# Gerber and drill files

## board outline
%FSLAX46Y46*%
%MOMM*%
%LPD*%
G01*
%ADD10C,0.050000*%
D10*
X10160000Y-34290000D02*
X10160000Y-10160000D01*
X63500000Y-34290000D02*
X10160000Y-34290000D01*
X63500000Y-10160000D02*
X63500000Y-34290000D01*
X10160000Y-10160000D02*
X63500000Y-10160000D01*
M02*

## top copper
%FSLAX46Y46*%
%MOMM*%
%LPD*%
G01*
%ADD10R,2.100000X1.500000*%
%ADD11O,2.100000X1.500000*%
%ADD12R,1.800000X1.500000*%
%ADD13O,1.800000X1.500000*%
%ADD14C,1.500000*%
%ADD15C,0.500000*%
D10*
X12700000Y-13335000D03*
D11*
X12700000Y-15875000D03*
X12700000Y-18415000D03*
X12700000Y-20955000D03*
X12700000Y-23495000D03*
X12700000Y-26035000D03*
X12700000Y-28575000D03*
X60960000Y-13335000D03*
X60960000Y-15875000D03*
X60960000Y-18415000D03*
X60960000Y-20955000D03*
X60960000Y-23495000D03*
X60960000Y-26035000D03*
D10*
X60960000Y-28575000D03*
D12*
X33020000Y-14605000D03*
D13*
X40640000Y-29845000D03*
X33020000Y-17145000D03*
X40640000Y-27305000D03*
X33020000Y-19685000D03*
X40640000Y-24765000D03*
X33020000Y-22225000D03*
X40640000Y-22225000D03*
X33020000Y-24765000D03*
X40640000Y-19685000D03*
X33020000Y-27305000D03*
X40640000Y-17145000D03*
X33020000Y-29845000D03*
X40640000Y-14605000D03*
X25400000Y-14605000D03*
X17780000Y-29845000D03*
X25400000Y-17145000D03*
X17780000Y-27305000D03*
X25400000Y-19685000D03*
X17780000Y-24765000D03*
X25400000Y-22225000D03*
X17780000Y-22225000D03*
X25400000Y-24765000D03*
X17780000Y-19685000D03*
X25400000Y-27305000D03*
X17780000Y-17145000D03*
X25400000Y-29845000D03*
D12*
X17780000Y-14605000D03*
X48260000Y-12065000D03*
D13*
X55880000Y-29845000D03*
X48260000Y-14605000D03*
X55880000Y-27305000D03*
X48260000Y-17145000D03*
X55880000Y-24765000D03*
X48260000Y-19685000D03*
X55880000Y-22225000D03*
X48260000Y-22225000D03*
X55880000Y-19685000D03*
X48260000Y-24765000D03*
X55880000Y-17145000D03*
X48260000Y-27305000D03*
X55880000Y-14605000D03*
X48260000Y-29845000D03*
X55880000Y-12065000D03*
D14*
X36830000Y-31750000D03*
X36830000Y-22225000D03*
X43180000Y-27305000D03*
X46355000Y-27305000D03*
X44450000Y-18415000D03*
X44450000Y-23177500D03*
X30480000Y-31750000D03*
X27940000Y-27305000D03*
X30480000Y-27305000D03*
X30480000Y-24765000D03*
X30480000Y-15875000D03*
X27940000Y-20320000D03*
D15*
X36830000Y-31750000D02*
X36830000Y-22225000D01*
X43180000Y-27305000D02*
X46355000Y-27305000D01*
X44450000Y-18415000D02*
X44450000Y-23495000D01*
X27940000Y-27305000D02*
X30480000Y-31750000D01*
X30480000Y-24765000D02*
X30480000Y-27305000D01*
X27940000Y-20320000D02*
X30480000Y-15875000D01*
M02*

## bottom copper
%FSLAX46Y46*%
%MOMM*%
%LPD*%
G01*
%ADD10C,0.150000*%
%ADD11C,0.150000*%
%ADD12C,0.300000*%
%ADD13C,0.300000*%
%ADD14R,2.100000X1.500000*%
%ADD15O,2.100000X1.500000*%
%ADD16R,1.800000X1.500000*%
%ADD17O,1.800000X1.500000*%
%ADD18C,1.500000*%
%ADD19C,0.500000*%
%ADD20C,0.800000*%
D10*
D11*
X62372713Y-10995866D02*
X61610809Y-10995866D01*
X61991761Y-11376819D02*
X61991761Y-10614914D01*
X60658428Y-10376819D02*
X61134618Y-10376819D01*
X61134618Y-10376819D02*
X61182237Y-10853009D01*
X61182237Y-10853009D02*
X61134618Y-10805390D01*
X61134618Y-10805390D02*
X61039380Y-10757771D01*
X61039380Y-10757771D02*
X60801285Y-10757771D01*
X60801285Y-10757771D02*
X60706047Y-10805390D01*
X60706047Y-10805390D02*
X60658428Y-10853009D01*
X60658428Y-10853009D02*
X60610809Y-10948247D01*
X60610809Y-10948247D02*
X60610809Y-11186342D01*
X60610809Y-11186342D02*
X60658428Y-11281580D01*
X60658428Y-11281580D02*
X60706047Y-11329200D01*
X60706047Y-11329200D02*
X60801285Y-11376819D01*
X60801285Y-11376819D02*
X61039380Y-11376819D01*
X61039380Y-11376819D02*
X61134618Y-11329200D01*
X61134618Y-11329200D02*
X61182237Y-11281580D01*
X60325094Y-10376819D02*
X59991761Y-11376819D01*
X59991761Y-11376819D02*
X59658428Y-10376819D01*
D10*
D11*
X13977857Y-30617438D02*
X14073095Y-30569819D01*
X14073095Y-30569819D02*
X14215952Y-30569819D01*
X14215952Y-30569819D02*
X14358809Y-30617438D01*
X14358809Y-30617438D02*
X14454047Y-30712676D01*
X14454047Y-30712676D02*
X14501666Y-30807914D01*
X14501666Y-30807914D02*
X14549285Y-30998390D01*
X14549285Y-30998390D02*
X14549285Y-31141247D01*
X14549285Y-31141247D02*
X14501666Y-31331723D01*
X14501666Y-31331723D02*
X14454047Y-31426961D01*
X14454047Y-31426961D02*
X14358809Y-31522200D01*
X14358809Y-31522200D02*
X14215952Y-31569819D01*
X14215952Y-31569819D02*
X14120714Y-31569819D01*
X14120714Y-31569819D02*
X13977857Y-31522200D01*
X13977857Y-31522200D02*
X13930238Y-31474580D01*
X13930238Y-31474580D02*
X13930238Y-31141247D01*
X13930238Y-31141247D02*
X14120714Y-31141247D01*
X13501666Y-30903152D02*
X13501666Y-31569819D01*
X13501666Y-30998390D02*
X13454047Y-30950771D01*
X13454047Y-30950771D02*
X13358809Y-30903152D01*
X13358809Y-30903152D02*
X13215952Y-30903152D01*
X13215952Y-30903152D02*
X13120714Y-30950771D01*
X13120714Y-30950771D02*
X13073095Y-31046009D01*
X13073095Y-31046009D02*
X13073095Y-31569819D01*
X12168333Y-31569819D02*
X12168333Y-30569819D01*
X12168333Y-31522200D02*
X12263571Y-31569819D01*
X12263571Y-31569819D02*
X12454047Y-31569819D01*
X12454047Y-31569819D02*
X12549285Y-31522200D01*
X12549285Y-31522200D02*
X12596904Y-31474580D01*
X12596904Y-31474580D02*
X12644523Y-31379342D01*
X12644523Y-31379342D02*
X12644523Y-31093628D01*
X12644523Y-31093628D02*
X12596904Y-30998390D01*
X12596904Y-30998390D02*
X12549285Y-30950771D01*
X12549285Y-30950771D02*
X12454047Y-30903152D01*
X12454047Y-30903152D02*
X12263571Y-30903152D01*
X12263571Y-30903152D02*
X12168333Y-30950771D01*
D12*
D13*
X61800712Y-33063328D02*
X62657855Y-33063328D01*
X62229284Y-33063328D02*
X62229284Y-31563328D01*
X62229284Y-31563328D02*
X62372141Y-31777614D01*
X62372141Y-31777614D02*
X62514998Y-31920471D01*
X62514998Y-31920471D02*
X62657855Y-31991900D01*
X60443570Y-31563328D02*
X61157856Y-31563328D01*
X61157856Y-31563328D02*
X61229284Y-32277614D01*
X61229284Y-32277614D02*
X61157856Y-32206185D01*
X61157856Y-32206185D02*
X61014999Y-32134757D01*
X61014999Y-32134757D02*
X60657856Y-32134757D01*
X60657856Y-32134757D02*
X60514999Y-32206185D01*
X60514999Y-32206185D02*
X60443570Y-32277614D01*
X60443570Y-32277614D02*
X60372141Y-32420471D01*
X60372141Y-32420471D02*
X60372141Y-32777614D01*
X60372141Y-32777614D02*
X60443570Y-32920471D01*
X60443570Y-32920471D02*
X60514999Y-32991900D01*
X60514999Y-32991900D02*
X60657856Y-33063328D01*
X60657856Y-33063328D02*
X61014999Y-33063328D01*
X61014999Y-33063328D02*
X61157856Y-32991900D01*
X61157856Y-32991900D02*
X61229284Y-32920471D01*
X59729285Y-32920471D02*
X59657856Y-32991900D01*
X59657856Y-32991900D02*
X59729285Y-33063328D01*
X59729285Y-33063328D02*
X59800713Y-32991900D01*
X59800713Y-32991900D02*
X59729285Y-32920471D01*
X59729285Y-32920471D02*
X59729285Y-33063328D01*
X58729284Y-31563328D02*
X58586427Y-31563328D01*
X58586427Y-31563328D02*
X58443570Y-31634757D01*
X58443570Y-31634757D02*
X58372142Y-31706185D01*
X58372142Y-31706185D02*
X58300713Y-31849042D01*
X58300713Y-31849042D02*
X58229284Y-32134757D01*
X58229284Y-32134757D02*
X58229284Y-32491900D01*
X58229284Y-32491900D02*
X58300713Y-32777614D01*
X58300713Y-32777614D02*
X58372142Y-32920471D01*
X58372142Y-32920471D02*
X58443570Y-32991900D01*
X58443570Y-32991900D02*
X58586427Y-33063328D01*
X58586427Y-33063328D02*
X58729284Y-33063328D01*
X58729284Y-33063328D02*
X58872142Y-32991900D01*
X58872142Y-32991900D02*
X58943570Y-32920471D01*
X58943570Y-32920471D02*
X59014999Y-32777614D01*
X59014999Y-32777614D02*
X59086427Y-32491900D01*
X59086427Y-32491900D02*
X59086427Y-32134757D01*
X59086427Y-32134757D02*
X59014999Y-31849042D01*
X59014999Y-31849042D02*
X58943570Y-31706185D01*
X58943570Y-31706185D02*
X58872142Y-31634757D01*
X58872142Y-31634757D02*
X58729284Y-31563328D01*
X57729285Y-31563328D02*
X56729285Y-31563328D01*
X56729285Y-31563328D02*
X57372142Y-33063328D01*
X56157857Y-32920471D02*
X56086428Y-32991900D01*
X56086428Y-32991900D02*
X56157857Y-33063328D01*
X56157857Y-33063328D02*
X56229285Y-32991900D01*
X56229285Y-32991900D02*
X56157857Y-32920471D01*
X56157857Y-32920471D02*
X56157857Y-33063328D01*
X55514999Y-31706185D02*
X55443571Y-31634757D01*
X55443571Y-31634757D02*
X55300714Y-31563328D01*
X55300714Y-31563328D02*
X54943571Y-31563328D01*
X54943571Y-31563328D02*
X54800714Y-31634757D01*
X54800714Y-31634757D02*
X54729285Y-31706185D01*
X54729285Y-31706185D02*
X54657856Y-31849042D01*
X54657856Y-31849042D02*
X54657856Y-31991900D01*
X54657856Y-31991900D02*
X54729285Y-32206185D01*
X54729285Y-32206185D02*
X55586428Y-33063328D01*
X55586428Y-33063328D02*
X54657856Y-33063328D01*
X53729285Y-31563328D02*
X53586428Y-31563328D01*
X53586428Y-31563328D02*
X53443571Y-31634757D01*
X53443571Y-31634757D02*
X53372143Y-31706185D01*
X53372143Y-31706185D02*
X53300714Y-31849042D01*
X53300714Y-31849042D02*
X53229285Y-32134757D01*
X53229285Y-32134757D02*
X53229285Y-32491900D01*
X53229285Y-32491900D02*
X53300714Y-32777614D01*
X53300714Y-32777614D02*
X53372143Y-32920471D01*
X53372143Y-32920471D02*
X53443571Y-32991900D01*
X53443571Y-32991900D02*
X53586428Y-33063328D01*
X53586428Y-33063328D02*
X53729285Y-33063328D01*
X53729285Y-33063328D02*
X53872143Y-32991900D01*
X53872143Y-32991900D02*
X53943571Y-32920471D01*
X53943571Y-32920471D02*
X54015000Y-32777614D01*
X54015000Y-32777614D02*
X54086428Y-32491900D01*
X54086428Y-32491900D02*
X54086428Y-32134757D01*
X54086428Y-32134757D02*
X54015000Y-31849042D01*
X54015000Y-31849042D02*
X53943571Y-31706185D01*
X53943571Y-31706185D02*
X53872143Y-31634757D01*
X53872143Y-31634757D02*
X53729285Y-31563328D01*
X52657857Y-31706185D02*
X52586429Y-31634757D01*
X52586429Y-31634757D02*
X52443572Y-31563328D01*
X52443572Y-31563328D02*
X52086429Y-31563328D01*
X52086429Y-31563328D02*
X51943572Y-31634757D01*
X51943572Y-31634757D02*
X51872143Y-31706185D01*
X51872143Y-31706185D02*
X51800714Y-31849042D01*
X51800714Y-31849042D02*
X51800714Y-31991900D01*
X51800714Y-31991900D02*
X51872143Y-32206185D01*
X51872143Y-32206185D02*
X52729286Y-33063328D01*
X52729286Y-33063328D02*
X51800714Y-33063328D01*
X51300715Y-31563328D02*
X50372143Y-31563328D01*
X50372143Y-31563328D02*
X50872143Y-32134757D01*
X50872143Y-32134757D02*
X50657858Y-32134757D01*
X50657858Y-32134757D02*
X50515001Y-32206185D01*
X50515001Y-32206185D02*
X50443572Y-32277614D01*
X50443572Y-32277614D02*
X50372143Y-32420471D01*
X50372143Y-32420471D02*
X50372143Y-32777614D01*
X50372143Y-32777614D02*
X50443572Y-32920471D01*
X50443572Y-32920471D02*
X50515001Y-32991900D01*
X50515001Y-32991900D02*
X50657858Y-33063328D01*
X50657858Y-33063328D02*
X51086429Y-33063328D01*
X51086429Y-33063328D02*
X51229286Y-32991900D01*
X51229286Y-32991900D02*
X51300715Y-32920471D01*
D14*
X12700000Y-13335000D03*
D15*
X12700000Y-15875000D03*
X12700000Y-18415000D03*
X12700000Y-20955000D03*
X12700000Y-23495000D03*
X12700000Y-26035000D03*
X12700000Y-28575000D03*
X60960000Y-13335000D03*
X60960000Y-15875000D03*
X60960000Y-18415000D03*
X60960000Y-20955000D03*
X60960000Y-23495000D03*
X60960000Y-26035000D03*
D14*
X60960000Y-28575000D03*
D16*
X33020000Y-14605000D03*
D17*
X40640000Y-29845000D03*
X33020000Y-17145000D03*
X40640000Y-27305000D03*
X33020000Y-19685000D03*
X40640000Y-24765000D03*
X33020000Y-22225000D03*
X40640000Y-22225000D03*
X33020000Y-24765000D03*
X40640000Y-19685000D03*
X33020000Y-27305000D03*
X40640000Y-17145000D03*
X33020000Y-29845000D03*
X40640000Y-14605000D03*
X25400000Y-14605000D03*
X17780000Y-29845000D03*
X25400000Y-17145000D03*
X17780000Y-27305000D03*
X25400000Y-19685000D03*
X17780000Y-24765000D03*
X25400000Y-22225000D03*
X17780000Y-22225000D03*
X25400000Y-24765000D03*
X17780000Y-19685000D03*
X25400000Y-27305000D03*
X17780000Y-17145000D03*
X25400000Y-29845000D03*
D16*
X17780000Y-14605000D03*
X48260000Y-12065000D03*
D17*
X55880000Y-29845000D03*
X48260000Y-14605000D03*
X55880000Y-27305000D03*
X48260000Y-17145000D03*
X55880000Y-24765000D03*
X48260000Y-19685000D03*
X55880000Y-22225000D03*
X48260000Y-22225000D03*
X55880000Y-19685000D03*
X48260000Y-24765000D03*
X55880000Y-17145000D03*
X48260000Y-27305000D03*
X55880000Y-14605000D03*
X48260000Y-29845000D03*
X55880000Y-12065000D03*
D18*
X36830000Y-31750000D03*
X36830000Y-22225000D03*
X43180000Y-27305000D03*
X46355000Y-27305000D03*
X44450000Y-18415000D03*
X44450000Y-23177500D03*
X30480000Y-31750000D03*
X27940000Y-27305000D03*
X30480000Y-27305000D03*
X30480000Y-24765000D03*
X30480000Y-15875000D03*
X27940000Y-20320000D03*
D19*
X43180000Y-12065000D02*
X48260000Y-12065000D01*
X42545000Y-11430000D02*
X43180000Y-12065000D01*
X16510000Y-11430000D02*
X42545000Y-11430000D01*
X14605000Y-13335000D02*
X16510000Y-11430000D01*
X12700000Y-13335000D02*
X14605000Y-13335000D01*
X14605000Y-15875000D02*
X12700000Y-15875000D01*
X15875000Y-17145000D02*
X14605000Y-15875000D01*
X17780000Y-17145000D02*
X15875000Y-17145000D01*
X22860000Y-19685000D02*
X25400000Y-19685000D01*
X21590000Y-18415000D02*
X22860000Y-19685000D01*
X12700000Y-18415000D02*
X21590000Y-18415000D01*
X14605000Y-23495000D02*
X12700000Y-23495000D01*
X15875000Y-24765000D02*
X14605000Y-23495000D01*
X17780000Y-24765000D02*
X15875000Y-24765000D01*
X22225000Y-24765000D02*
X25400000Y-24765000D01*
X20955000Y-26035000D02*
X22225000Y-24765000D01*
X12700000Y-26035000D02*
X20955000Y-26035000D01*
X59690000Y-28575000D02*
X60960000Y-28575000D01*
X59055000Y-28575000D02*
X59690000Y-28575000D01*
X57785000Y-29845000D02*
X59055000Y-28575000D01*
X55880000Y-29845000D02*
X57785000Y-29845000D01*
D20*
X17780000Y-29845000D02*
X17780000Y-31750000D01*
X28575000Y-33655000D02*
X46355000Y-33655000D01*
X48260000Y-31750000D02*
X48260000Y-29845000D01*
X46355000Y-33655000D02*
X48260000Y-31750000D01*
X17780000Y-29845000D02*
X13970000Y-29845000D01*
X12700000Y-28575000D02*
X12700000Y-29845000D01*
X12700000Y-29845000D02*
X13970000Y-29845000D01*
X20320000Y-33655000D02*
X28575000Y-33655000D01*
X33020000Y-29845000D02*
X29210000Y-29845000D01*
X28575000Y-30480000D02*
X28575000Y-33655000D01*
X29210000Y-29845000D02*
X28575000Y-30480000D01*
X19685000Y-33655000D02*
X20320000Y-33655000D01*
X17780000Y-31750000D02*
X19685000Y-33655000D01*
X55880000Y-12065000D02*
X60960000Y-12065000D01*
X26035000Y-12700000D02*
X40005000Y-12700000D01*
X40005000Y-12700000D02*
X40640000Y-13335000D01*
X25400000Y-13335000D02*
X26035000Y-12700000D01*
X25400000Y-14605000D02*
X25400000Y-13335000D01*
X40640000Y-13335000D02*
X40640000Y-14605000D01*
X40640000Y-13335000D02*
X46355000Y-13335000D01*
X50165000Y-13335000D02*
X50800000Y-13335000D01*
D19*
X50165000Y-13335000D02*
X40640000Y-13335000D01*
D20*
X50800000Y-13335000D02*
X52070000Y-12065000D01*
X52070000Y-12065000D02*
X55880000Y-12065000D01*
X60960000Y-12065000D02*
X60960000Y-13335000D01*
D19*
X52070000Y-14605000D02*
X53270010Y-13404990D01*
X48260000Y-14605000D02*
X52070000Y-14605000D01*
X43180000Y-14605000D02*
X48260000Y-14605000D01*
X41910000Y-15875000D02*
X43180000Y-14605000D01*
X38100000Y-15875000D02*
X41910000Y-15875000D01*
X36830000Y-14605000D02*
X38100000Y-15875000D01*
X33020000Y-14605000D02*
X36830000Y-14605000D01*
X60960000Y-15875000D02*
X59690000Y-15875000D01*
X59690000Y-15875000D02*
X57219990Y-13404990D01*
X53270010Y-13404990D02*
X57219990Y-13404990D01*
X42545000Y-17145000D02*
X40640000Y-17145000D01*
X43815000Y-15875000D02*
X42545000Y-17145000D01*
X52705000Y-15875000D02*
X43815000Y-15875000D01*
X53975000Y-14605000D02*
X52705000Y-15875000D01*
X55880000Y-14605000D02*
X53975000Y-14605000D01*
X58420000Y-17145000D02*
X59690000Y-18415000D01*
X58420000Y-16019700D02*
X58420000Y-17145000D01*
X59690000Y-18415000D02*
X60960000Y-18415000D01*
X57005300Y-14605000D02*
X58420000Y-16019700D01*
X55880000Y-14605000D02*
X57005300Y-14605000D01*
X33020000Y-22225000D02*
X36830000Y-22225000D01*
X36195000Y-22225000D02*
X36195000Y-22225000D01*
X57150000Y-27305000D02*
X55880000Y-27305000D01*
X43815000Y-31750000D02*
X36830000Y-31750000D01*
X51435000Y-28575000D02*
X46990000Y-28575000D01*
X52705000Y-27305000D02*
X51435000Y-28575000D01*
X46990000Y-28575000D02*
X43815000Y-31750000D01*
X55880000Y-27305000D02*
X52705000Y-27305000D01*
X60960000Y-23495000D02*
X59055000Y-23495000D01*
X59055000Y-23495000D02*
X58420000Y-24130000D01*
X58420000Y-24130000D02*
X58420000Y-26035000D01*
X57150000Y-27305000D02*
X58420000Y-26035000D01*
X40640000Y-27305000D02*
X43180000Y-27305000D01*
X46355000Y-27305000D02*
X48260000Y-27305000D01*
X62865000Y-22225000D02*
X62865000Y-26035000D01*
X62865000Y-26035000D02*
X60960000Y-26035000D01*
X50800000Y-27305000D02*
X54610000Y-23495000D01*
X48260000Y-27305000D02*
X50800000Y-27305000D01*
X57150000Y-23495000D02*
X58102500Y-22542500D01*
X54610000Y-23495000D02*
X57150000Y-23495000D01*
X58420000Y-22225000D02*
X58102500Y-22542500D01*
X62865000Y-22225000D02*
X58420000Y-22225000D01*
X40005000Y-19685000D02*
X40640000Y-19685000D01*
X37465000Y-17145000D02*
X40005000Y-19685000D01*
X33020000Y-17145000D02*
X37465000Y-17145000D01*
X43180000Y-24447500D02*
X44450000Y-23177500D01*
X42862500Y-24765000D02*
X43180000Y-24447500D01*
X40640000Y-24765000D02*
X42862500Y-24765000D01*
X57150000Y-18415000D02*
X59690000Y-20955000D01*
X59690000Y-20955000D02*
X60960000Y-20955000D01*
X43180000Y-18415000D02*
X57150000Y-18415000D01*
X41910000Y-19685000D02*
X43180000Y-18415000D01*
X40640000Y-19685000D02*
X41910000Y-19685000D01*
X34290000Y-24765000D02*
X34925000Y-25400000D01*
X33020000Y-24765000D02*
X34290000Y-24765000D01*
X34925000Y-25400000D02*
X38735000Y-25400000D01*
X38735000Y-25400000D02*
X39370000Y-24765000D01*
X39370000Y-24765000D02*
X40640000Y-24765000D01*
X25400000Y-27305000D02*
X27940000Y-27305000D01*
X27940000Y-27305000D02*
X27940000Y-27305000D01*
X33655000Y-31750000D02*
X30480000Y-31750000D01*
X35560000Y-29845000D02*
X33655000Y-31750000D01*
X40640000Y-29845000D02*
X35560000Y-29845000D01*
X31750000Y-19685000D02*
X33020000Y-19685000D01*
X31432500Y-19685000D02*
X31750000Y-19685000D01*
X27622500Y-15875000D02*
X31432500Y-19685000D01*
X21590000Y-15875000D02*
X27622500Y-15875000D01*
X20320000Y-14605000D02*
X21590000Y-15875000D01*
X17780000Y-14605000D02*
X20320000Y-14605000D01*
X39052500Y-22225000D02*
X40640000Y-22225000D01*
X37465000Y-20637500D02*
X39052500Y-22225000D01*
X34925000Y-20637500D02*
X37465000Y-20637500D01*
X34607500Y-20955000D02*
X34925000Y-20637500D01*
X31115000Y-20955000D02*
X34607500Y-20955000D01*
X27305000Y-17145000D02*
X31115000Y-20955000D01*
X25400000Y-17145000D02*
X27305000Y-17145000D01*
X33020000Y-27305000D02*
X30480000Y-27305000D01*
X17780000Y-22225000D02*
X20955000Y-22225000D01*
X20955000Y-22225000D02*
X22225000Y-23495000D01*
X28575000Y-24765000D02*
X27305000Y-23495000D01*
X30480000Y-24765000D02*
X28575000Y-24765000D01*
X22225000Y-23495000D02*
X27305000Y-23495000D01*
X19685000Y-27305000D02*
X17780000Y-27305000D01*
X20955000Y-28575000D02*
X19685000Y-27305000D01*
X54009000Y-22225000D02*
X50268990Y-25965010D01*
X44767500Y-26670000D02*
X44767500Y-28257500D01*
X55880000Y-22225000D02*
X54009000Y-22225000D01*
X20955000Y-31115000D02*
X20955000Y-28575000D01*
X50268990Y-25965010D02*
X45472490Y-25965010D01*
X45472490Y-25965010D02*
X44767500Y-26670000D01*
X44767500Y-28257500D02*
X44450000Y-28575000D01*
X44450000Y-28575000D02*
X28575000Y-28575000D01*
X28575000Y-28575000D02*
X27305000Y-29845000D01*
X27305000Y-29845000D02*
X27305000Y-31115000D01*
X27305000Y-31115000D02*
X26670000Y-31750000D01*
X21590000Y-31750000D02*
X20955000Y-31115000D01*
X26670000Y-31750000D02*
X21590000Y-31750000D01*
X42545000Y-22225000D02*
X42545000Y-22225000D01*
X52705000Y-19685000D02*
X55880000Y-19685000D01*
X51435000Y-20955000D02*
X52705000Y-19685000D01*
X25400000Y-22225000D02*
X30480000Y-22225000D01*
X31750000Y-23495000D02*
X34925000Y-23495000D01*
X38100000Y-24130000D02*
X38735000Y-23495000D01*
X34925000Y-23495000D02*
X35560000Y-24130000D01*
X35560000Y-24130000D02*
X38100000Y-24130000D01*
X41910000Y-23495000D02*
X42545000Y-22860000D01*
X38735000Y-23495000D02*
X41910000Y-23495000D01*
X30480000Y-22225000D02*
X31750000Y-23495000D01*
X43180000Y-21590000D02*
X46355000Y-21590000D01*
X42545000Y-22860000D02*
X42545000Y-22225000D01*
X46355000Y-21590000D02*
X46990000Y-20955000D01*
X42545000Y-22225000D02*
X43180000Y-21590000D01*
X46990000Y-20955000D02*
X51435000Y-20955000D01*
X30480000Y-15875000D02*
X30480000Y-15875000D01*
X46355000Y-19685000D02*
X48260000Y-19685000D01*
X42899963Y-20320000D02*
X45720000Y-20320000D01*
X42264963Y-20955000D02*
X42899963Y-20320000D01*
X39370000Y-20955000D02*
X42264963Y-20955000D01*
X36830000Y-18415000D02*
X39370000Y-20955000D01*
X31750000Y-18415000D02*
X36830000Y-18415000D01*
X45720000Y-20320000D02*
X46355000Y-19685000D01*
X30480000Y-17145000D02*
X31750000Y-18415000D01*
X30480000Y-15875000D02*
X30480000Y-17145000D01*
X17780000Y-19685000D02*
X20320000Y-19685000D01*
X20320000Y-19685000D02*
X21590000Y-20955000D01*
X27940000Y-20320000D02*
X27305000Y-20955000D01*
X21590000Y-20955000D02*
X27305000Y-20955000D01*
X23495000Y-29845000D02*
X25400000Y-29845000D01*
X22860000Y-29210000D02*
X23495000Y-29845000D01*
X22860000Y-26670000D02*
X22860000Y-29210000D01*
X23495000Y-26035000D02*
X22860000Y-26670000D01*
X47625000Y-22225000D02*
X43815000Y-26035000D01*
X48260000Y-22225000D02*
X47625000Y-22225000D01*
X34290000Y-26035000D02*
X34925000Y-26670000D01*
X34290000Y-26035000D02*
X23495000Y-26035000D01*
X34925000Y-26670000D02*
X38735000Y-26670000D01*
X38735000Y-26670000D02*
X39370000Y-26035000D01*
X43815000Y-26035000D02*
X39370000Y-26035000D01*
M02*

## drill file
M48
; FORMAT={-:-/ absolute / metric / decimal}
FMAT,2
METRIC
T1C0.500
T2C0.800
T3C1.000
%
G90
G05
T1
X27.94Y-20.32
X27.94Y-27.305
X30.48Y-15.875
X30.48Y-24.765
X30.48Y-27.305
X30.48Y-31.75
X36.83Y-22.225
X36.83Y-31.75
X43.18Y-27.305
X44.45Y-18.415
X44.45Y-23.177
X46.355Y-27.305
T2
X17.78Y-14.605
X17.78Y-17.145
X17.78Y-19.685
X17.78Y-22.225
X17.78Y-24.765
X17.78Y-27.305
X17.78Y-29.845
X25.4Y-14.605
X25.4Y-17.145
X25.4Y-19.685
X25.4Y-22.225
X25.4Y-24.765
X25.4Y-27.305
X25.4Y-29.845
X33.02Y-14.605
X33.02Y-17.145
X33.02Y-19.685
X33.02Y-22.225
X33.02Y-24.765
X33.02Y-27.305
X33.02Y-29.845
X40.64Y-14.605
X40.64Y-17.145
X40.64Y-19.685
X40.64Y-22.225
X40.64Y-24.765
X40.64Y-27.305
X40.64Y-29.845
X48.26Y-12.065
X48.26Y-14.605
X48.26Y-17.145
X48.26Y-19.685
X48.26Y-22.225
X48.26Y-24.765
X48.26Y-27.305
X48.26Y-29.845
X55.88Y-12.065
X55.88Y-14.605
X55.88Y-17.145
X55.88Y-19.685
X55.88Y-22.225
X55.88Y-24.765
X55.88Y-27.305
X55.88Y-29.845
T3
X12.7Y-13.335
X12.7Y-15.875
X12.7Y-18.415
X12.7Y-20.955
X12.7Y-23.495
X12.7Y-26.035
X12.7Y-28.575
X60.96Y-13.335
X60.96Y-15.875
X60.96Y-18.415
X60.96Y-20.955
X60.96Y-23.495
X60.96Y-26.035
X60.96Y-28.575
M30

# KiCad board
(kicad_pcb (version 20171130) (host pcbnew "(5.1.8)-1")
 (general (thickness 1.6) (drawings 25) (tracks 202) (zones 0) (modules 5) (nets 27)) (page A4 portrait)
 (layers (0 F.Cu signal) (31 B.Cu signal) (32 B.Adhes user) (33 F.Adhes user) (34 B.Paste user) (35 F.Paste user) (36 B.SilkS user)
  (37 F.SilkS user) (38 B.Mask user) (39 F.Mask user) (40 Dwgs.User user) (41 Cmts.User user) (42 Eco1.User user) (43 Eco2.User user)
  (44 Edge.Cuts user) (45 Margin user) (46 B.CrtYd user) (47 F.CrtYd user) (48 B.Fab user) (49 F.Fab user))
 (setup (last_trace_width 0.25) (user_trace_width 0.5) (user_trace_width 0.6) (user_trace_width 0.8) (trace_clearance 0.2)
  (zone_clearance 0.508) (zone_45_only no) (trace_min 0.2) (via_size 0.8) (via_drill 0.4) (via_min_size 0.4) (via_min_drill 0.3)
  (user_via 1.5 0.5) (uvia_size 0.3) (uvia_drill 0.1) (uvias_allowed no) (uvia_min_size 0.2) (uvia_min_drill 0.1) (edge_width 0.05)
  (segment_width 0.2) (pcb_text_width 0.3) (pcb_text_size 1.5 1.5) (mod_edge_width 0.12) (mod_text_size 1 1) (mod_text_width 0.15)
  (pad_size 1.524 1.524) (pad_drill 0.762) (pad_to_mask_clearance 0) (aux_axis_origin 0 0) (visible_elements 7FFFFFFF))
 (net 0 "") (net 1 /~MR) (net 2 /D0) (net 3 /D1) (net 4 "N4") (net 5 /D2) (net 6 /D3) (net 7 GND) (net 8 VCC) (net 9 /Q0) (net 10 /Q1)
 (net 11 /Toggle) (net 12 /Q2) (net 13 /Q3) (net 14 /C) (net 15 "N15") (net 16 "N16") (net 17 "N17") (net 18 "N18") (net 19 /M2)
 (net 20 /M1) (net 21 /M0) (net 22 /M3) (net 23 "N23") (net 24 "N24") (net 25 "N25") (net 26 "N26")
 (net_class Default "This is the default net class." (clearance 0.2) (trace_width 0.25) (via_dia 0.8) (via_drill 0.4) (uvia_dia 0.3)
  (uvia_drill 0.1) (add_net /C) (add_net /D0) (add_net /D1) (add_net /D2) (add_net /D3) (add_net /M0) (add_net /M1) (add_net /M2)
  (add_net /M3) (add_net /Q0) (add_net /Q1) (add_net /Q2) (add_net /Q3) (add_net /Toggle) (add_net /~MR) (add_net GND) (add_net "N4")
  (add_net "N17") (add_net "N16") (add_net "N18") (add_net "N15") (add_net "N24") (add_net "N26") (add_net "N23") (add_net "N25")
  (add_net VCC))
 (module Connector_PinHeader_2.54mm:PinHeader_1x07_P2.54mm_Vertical (layer B.Cu) (at 12.7 13.335 180)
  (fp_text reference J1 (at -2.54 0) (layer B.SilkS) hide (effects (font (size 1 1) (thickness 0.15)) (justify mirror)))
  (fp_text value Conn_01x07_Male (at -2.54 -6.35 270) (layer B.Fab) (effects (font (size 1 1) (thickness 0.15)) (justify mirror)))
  (pad 1 thru_hole rect (at 0 0 180) (size 2.1 1.5) (drill 1) (layers *.Cu *.Mask) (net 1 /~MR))
  (pad 2 thru_hole oval (at 0 -2.54 180) (size 2.1 1.5) (drill 1) (layers *.Cu *.Mask) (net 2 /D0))
  (pad 3 thru_hole oval (at 0 -5.08 180) (size 2.1 1.5) (drill 1) (layers *.Cu *.Mask) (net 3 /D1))
  (pad 4 thru_hole oval (at 0 -7.62 180) (size 2.1 1.5) (drill 1) (layers *.Cu *.Mask) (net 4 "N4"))
  (pad 5 thru_hole oval (at 0 -10.16 180) (size 2.1 1.5) (drill 1) (layers *.Cu *.Mask) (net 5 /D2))
  (pad 6 thru_hole oval (at 0 -12.7 180) (size 2.1 1.5) (drill 1) (layers *.Cu *.Mask) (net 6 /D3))
  (pad 7 thru_hole oval (at 0 -15.24 180) (size 2.1 1.5) (drill 1) (layers *.Cu *.Mask) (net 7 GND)))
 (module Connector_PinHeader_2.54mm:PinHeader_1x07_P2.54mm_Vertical (layer B.Cu) (at 60.96 28.575)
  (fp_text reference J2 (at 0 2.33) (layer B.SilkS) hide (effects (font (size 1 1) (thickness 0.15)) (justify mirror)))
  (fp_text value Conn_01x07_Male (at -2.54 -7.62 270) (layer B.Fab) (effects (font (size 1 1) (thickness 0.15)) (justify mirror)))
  (pad 7 thru_hole oval (at 0 -15.24) (size 2.1 1.5) (drill 1) (layers *.Cu *.Mask) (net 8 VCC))
  (pad 6 thru_hole oval (at 0 -12.7) (size 2.1 1.5) (drill 1) (layers *.Cu *.Mask) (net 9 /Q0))
  (pad 5 thru_hole oval (at 0 -10.16) (size 2.1 1.5) (drill 1) (layers *.Cu *.Mask) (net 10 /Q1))
  (pad 4 thru_hole oval (at 0 -7.62) (size 2.1 1.5) (drill 1) (layers *.Cu *.Mask) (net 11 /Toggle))
  (pad 3 thru_hole oval (at 0 -5.08) (size 2.1 1.5) (drill 1) (layers *.Cu *.Mask) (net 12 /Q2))
  (pad 2 thru_hole oval (at 0 -2.54) (size 2.1 1.5) (drill 1) (layers *.Cu *.Mask) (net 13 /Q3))
  (pad 1 thru_hole rect (at 0 0) (size 2.1 1.5) (drill 1) (layers *.Cu *.Mask) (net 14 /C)))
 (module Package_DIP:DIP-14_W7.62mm (layer F.Cu) (at 33.02 14.605)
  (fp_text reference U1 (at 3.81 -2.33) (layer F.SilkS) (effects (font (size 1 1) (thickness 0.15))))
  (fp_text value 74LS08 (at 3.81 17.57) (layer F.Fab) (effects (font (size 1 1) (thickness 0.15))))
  (pad 1 thru_hole rect (at 0 0) (size 1.8 1.5) (drill 0.8) (layers *.Cu *.Mask) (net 9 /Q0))
  (pad 8 thru_hole oval (at 7.62 15.24) (size 1.8 1.5) (drill 0.8) (layers *.Cu *.Mask) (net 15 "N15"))
  (pad 2 thru_hole oval (at 0 2.54) (size 1.8 1.5) (drill 0.8) (layers *.Cu *.Mask) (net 11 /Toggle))
  (pad 9 thru_hole oval (at 7.62 12.7) (size 1.8 1.5) (drill 0.8) (layers *.Cu *.Mask) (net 13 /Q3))
  (pad 3 thru_hole oval (at 0 5.08) (size 1.8 1.5) (drill 0.8) (layers *.Cu *.Mask) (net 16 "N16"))
  (pad 10 thru_hole oval (at 7.62 10.16) (size 1.8 1.5) (drill 0.8) (layers *.Cu *.Mask) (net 11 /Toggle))
  (pad 4 thru_hole oval (at 0 7.62) (size 1.8 1.5) (drill 0.8) (layers *.Cu *.Mask) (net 12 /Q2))
  (pad 11 thru_hole oval (at 7.62 7.62) (size 1.8 1.5) (drill 0.8) (layers *.Cu *.Mask) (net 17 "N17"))
  (pad 5 thru_hole oval (at 0 10.16) (size 1.8 1.5) (drill 0.8) (layers *.Cu *.Mask) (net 11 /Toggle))
  (pad 12 thru_hole oval (at 7.62 5.08) (size 1.8 1.5) (drill 0.8) (layers *.Cu *.Mask) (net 11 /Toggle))
  (pad 6 thru_hole oval (at 0 12.7) (size 1.8 1.5) (drill 0.8) (layers *.Cu *.Mask) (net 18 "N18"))
  (pad 13 thru_hole oval (at 7.62 2.54) (size 1.8 1.5) (drill 0.8) (layers *.Cu *.Mask) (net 10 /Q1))
  (pad 7 thru_hole oval (at 0 15.24) (size 1.8 1.5) (drill 0.8) (layers *.Cu *.Mask) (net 7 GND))
  (pad 14 thru_hole oval (at 7.62 0) (size 1.8 1.5) (drill 0.8) (layers *.Cu *.Mask) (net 8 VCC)))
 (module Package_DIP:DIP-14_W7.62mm (layer F.Cu) (at 17.78 14.605)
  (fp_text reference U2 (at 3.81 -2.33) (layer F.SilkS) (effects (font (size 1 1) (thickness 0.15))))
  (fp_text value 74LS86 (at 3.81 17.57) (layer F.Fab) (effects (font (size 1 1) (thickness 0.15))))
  (pad 14 thru_hole oval (at 7.62 0) (size 1.8 1.5) (drill 0.8) (layers *.Cu *.Mask) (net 8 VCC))
  (pad 7 thru_hole oval (at 0 15.24) (size 1.8 1.5) (drill 0.8) (layers *.Cu *.Mask) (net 7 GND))
  (pad 13 thru_hole oval (at 7.62 2.54) (size 1.8 1.5) (drill 0.8) (layers *.Cu *.Mask) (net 17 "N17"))
  (pad 6 thru_hole oval (at 0 12.7) (size 1.8 1.5) (drill 0.8) (layers *.Cu *.Mask) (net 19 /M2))
  (pad 12 thru_hole oval (at 7.62 5.08) (size 1.8 1.5) (drill 0.8) (layers *.Cu *.Mask) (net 3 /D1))
  (pad 5 thru_hole oval (at 0 10.16) (size 1.8 1.5) (drill 0.8) (layers *.Cu *.Mask) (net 5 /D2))
  (pad 11 thru_hole oval (at 7.62 7.62) (size 1.8 1.5) (drill 0.8) (layers *.Cu *.Mask) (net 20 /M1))
  (pad 4 thru_hole oval (at 0 7.62) (size 1.8 1.5) (drill 0.8) (layers *.Cu *.Mask) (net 18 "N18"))
  (pad 10 thru_hole oval (at 7.62 10.16) (size 1.8 1.5) (drill 0.8) (layers *.Cu *.Mask) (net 6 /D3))
  (pad 3 thru_hole oval (at 0 5.08) (size 1.8 1.5) (drill 0.8) (layers *.Cu *.Mask) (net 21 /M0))
  (pad 9 thru_hole oval (at 7.62 12.7) (size 1.8 1.5) (drill 0.8) (layers *.Cu *.Mask) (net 15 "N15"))
  (pad 2 thru_hole oval (at 0 2.54) (size 1.8 1.5) (drill 0.8) (layers *.Cu *.Mask) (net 2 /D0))
  (pad 8 thru_hole oval (at 7.62 15.24) (size 1.8 1.5) (drill 0.8) (layers *.Cu *.Mask) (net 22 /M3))
  (pad 1 thru_hole rect (at 0 0) (size 1.8 1.5) (drill 0.8) (layers *.Cu *.Mask) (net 16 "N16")))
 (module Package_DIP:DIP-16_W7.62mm (layer F.Cu) (at 48.26 12.065)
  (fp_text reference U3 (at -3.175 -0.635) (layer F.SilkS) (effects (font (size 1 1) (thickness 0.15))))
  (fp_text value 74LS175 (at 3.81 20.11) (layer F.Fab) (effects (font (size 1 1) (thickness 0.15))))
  (pad 1 thru_hole rect (at 0 0) (size 1.8 1.5) (drill 0.8) (layers *.Cu *.Mask) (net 1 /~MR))
  (pad 9 thru_hole oval (at 7.62 17.78) (size 1.8 1.5) (drill 0.8) (layers *.Cu *.Mask) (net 14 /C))
  (pad 2 thru_hole oval (at 0 2.54) (size 1.8 1.5) (drill 0.8) (layers *.Cu *.Mask) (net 9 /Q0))
  (pad 10 thru_hole oval (at 7.62 15.24) (size 1.8 1.5) (drill 0.8) (layers *.Cu *.Mask) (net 12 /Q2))
  (pad 3 thru_hole oval (at 0 5.08) (size 1.8 1.5) (drill 0.8) (layers *.Cu *.Mask) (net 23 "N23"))
  (pad 11 thru_hole oval (at 7.62 12.7) (size 1.8 1.5) (drill 0.8) (layers *.Cu *.Mask) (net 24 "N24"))
  (pad 4 thru_hole oval (at 0 7.62) (size 1.8 1.5) (drill 0.8) (layers *.Cu *.Mask) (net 21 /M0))
  (pad 12 thru_hole oval (at 7.62 10.16) (size 1.8 1.5) (drill 0.8) (layers *.Cu *.Mask) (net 19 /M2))
  (pad 5 thru_hole oval (at 0 10.16) (size 1.8 1.5) (drill 0.8) (layers *.Cu *.Mask) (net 22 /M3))
  (pad 13 thru_hole oval (at 7.62 7.62) (size 1.8 1.5) (drill 0.8) (layers *.Cu *.Mask) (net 20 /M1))
  (pad 6 thru_hole oval (at 0 12.7) (size 1.8 1.5) (drill 0.8) (layers *.Cu *.Mask) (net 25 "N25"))
  (pad 14 thru_hole oval (at 7.62 5.08) (size 1.8 1.5) (drill 0.8) (layers *.Cu *.Mask) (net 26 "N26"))
  (pad 7 thru_hole oval (at 0 15.24) (size 1.8 1.5) (drill 0.8) (layers *.Cu *.Mask) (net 13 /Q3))
  (pad 15 thru_hole oval (at 7.62 2.54) (size 1.8 1.5) (drill 0.8) (layers *.Cu *.Mask) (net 10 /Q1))
  (pad 8 thru_hole oval (at 0 17.78) (size 1.8 1.5) (drill 0.8) (layers *.Cu *.Mask) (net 7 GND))
  (pad 16 thru_hole oval (at 7.62 0) (size 1.8 1.5) (drill 0.8) (layers *.Cu *.Mask) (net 8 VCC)))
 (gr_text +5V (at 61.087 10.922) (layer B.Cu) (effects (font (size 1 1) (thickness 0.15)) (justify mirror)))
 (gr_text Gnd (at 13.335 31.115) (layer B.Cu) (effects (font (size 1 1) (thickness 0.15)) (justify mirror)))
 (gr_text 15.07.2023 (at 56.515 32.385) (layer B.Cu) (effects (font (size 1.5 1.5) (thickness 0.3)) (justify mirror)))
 (gr_line (start 10.16 34.29) (end 10.16 10.16) (layer Edge.Cuts) (width 0.05))
 (gr_line (start 63.5 34.29) (end 10.16 34.29) (layer Edge.Cuts) (width 0.05))
 (gr_line (start 63.5 10.16) (end 63.5 34.29) (layer Edge.Cuts) (width 0.05))
 (gr_line (start 10.16 10.16) (end 63.5 10.16) (layer Edge.Cuts) (width 0.05))
 (segment (start 43.18 12.065) (end 48.26 12.065) (width 0.5) (layer B.Cu) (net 1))
 (segment (start 42.545 11.43) (end 43.18 12.065) (width 0.5) (layer B.Cu) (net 1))
 (segment (start 16.51 11.43) (end 42.545 11.43) (width 0.5) (layer B.Cu) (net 1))
 (segment (start 14.605 13.335) (end 16.51 11.43) (width 0.5) (layer B.Cu) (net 1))
 (segment (start 12.7 13.335) (end 14.605 13.335) (width 0.5) (layer B.Cu) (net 1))
 (segment (start 14.605 15.875) (end 12.7 15.875) (width 0.5) (layer B.Cu) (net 2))
 (segment (start 15.875 17.145) (end 14.605 15.875) (width 0.5) (layer B.Cu) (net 2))
 (segment (start 17.78 17.145) (end 15.875 17.145) (width 0.5) (layer B.Cu) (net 2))
 (segment (start 22.86 19.685) (end 25.4 19.685) (width 0.5) (layer B.Cu) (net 3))
 (segment (start 21.59 18.415) (end 22.86 19.685) (width 0.5) (layer B.Cu) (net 3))
 (segment (start 12.7 18.415) (end 21.59 18.415) (width 0.5) (layer B.Cu) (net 3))
 (segment (start 14.605 23.495) (end 12.7 23.495) (width 0.5) (layer B.Cu) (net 5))
 (segment (start 15.875 24.765) (end 14.605 23.495) (width 0.5) (layer B.Cu) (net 5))
 (segment (start 17.78 24.765) (end 15.875 24.765) (width 0.5) (layer B.Cu) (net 5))
 (segment (start 22.225 24.765) (end 25.4 24.765) (width 0.5) (layer B.Cu) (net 6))
 (segment (start 20.955 26.035) (end 22.225 24.765) (width 0.5) (layer B.Cu) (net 6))
 (segment (start 12.7 26.035) (end 20.955 26.035) (width 0.5) (layer B.Cu) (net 6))
 (segment (start 59.69 28.575) (end 60.96 28.575) (width 0.5) (layer B.Cu) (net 14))
 (segment (start 59.055 28.575) (end 59.69 28.575) (width 0.5) (layer B.Cu) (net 14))
 (segment (start 57.785 29.845) (end 59.055 28.575) (width 0.5) (layer B.Cu) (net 14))
 (segment (start 55.88 29.845) (end 57.785 29.845) (width 0.5) (layer B.Cu) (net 14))
 (segment (start 17.78 29.845) (end 17.78 31.75) (width 0.8) (layer B.Cu) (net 7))
 (segment (start 28.575 33.655) (end 46.355 33.655) (width 0.8) (layer B.Cu) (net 7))
 (segment (start 48.26 31.75) (end 48.26 29.845) (width 0.8) (layer B.Cu) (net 7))
 (segment (start 46.355 33.655) (end 48.26 31.75) (width 0.8) (layer B.Cu) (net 7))
 (segment (start 17.78 29.845) (end 13.97 29.845) (width 0.8) (layer B.Cu) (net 7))
 (segment (start 12.7 28.575) (end 12.7 29.845) (width 0.8) (layer B.Cu) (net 7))
 (segment (start 12.7 29.845) (end 13.97 29.845) (width 0.8) (layer B.Cu) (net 7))
 (segment (start 20.32 33.655) (end 28.575 33.655) (width 0.8) (layer B.Cu) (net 7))
 (segment (start 33.02 29.845) (end 29.21 29.845) (width 0.8) (layer B.Cu) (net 7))
 (segment (start 28.575 30.48) (end 28.575 33.655) (width 0.8) (layer B.Cu) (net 7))
 (segment (start 29.21 29.845) (end 28.575 30.48) (width 0.8) (layer B.Cu) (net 7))
 (segment (start 19.685 33.655) (end 20.32 33.655) (width 0.8) (layer B.Cu) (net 7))
 (segment (start 17.78 31.75) (end 19.685 33.655) (width 0.8) (layer B.Cu) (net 7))
 (segment (start 55.88 12.065) (end 60.96 12.065) (width 0.8) (layer B.Cu) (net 8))
 (segment (start 26.035 12.7) (end 40.005 12.7) (width 0.8) (layer B.Cu) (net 8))
 (segment (start 40.005 12.7) (end 40.64 13.335) (width 0.8) (layer B.Cu) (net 8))
 (segment (start 25.4 13.335) (end 26.035 12.7) (width 0.8) (layer B.Cu) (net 8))
 (segment (start 25.4 14.605) (end 25.4 13.335) (width 0.8) (layer B.Cu) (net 8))
 (segment (start 40.64 13.335) (end 40.64 14.605) (width 0.8) (layer B.Cu) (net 8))
 (segment (start 40.64 13.335) (end 46.355 13.335) (width 0.8) (layer B.Cu) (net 8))
 (segment (start 50.165 13.335) (end 50.8 13.335) (width 0.8) (layer B.Cu) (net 8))
 (segment (start 50.165 13.335) (end 40.64 13.335) (width 0.5) (layer B.Cu) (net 8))
 (segment (start 50.8 13.335) (end 52.07 12.065) (width 0.8) (layer B.Cu) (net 8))
 (segment (start 52.07 12.065) (end 55.88 12.065) (width 0.8) (layer B.Cu) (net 8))
 (segment (start 60.96 12.065) (end 60.96 13.335) (width 0.8) (layer B.Cu) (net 8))
 (segment (start 52.07 14.605) (end 53.27001 13.40499) (width 0.5) (layer B.Cu) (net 9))
 (segment (start 48.26 14.605) (end 52.07 14.605) (width 0.5) (layer B.Cu) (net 9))
 (segment (start 43.18 14.605) (end 48.26 14.605) (width 0.5) (layer B.Cu) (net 9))
 (segment (start 41.91 15.875) (end 43.18 14.605) (width 0.5) (layer B.Cu) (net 9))
 (segment (start 38.1 15.875) (end 41.91 15.875) (width 0.5) (layer B.Cu) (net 9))
 (segment (start 36.83 14.605) (end 38.1 15.875) (width 0.5) (layer B.Cu) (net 9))
 (segment (start 33.02 14.605) (end 36.83 14.605) (width 0.5) (layer B.Cu) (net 9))
 (segment (start 60.96 15.875) (end 59.69 15.875) (width 0.5) (layer B.Cu) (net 9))
 (segment (start 59.69 15.875) (end 57.21999 13.40499) (width 0.5) (layer B.Cu) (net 9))
 (segment (start 53.27001 13.40499) (end 57.21999 13.40499) (width 0.5) (layer B.Cu) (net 9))
 (segment (start 42.545 17.145) (end 40.64 17.145) (width 0.5) (layer B.Cu) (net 10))
 (segment (start 43.815 15.875) (end 42.545 17.145) (width 0.5) (layer B.Cu) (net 10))
 (segment (start 52.705 15.875) (end 43.815 15.875) (width 0.5) (layer B.Cu) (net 10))
 (segment (start 53.975 14.605) (end 52.705 15.875) (width 0.5) (layer B.Cu) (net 10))
 (segment (start 55.88 14.605) (end 53.975 14.605) (width 0.5) (layer B.Cu) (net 10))
 (segment (start 58.42 17.145) (end 59.69 18.415) (width 0.5) (layer B.Cu) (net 10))
 (segment (start 58.42 16.0197) (end 58.42 17.145) (width 0.5) (layer B.Cu) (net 10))
 (segment (start 59.69 18.415) (end 60.96 18.415) (width 0.5) (layer B.Cu) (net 10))
 (segment (start 57.0053 14.605) (end 58.42 16.0197) (width 0.5) (layer B.Cu) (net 10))
 (segment (start 55.88 14.605) (end 57.0053 14.605) (width 0.5) (layer B.Cu) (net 10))
 (via (at 36.83 31.75) (size 1.5) (drill 0.5) (layers F.Cu B.Cu) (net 12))
 (segment (start 33.02 22.225) (end 36.83 22.225) (width 0.5) (layer B.Cu) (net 12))
 (segment (start 36.195 22.225) (end 36.195 22.225) (width 0.5) (layer B.Cu) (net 12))
 (via (at 36.83 22.225) (size 1.5) (drill 0.5) (layers F.Cu B.Cu) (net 12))
 (segment (start 36.83 31.75) (end 36.83 22.225) (width 0.5) (layer F.Cu) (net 12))
 (segment (start 57.15 27.305) (end 55.88 27.305) (width 0.5) (layer B.Cu) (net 12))
 (segment (start 43.815 31.75) (end 36.83 31.75) (width 0.5) (layer B.Cu) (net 12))
 (segment (start 51.435 28.575) (end 46.99 28.575) (width 0.5) (layer B.Cu) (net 12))
 (segment (start 52.705 27.305) (end 51.435 28.575) (width 0.5) (layer B.Cu) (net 12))
 (segment (start 46.99 28.575) (end 43.815 31.75) (width 0.5) (layer B.Cu) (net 12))
 (segment (start 55.88 27.305) (end 52.705 27.305) (width 0.5) (layer B.Cu) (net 12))
 (segment (start 60.96 23.495) (end 59.055 23.495) (width 0.5) (layer B.Cu) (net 12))
 (segment (start 59.055 23.495) (end 58.42 24.13) (width 0.5) (layer B.Cu) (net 12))
 (segment (start 58.42 24.13) (end 58.42 26.035) (width 0.5) (layer B.Cu) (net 12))
 (segment (start 57.15 27.305) (end 58.42 26.035) (width 0.5) (layer B.Cu) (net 12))
 (segment (start 40.64 27.305) (end 43.18 27.305) (width 0.5) (layer B.Cu) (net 13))
 (segment (start 43.18 27.305) (end 46.355 27.305) (width 0.5) (layer F.Cu) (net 13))
 (via (at 43.18 27.305) (size 1.5) (drill 0.5) (layers F.Cu B.Cu) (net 13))
 (segment (start 46.355 27.305) (end 48.26 27.305) (width 0.5) (layer B.Cu) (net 13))
 (via (at 46.355 27.305) (size 1.5) (drill 0.5) (layers F.Cu B.Cu) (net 13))
 (segment (start 62.865 22.225) (end 62.865 26.035) (width 0.5) (layer B.Cu) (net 13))
 (segment (start 62.865 26.035) (end 60.96 26.035) (width 0.5) (layer B.Cu) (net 13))
 (segment (start 50.8 27.305) (end 54.61 23.495) (width 0.5) (layer B.Cu) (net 13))
 (segment (start 48.26 27.305) (end 50.8 27.305) (width 0.5) (layer B.Cu) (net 13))
 (segment (start 57.15 23.495) (end 58.1025 22.5425) (width 0.5) (layer B.Cu) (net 13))
 (segment (start 54.61 23.495) (end 57.15 23.495) (width 0.5) (layer B.Cu) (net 13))
 (segment (start 58.42 22.225) (end 58.1025 22.5425) (width 0.5) (layer B.Cu) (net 13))
 (segment (start 62.865 22.225) (end 58.42 22.225) (width 0.5) (layer B.Cu) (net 13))
 (segment (start 44.45 18.415) (end 44.45 23.495) (width 0.5) (layer F.Cu) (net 11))
 (via (at 44.45 18.415) (size 1.5) (drill 0.5) (layers F.Cu B.Cu) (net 11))
 (via (at 44.45 23.1775) (size 1.5) (drill 0.5) (layers F.Cu B.Cu) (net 11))
 (segment (start 40.005 19.685) (end 40.64 19.685) (width 0.5) (layer B.Cu) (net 11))
 (segment (start 37.465 17.145) (end 40.005 19.685) (width 0.5) (layer B.Cu) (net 11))
 (segment (start 33.02 17.145) (end 37.465 17.145) (width 0.5) (layer B.Cu) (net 11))
 (segment (start 43.18 24.4475) (end 44.45 23.1775) (width 0.5) (layer B.Cu) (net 11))
 (segment (start 42.8625 24.765) (end 43.18 24.4475) (width 0.5) (layer B.Cu) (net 11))
 (segment (start 40.64 24.765) (end 42.8625 24.765) (width 0.5) (layer B.Cu) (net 11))
 (segment (start 57.15 18.415) (end 59.69 20.955) (width 0.5) (layer B.Cu) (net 11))
 (segment (start 59.69 20.955) (end 60.96 20.955) (width 0.5) (layer B.Cu) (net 11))
 (segment (start 43.18 18.415) (end 57.15 18.415) (width 0.5) (layer B.Cu) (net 11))
 (segment (start 41.91 19.685) (end 43.18 18.415) (width 0.5) (layer B.Cu) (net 11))
 (segment (start 40.64 19.685) (end 41.91 19.685) (width 0.5) (layer B.Cu) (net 11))
 (segment (start 34.29 24.765) (end 34.925 25.4) (width 0.5) (layer B.Cu) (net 11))
 (segment (start 33.02 24.765) (end 34.29 24.765) (width 0.5) (layer B.Cu) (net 11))
 (segment (start 34.925 25.4) (end 38.735 25.4) (width 0.5) (layer B.Cu) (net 11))
 (segment (start 38.735 25.4) (end 39.37 24.765) (width 0.5) (layer B.Cu) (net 11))
 (segment (start 39.37 24.765) (end 40.64 24.765) (width 0.5) (layer B.Cu) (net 11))
 (via (at 30.48 31.75) (size 1.5) (drill 0.5) (layers F.Cu B.Cu) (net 15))
 (segment (start 25.4 27.305) (end 27.94 27.305) (width 0.5) (layer B.Cu) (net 15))
 (segment (start 27.94 27.305) (end 27.94 27.305) (width 0.5) (layer B.Cu) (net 15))
 (via (at 27.94 27.305) (size 1.5) (drill 0.5) (layers F.Cu B.Cu) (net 15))
 (segment (start 27.94 27.305) (end 30.48 31.75) (width 0.5) (layer F.Cu) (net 15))
 (segment (start 33.655 31.75) (end 30.48 31.75) (width 0.5) (layer B.Cu) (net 15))
 (segment (start 35.56 29.845) (end 33.655 31.75) (width 0.5) (layer B.Cu) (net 15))
 (segment (start 40.64 29.845) (end 35.56 29.845) (width 0.5) (layer B.Cu) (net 15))
 (segment (start 31.75 19.685) (end 33.02 19.685) (width 0.5) (layer B.Cu) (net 16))
 (segment (start 31.4325 19.685) (end 31.75 19.685) (width 0.5) (layer B.Cu) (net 16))
 (segment (start 27.6225 15.875) (end 31.4325 19.685) (width 0.5) (layer B.Cu) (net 16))
 (segment (start 21.59 15.875) (end 27.6225 15.875) (width 0.5) (layer B.Cu) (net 16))
 (segment (start 20.32 14.605) (end 21.59 15.875) (width 0.5) (layer B.Cu) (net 16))
 (segment (start 17.78 14.605) (end 20.32 14.605) (width 0.5) (layer B.Cu) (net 16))
 (segment (start 39.0525 22.225) (end 40.64 22.225) (width 0.5) (layer B.Cu) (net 17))
 (segment (start 37.465 20.6375) (end 39.0525 22.225) (width 0.5) (layer B.Cu) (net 17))
 (segment (start 34.925 20.6375) (end 37.465 20.6375) (width 0.5) (layer B.Cu) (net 17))
 (segment (start 34.6075 20.955) (end 34.925 20.6375) (width 0.5) (layer B.Cu) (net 17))
 (segment (start 31.115 20.955) (end 34.6075 20.955) (width 0.5) (layer B.Cu) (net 17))
 (segment (start 27.305 17.145) (end 31.115 20.955) (width 0.5) (layer B.Cu) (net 17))
 (segment (start 25.4 17.145) (end 27.305 17.145) (width 0.5) (layer B.Cu) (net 17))
 (segment (start 33.02 27.305) (end 30.48 27.305) (width 0.5) (layer B.Cu) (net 18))
 (via (at 30.48 27.305) (size 1.5) (drill 0.5) (layers F.Cu B.Cu) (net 18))
 (segment (start 17.78 22.225) (end 20.955 22.225) (width 0.5) (layer B.Cu) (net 18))
 (segment (start 20.955 22.225) (end 22.225 23.495) (width 0.5) (layer B.Cu) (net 18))
 (via (at 30.48 24.765) (size 1.5) (drill 0.5) (layers F.Cu B.Cu) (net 18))
 (segment (start 30.48 24.765) (end 30.48 27.305) (width 0.5) (layer F.Cu) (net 18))
 (segment (start 28.575 24.765) (end 27.305 23.495) (width 0.5) (layer B.Cu) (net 18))
 (segment (start 30.48 24.765) (end 28.575 24.765) (width 0.5) (layer B.Cu) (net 18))
 (segment (start 22.225 23.495) (end 27.305 23.495) (width 0.5) (layer B.Cu) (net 18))
 (segment (start 19.685 27.305) (end 17.78 27.305) (width 0.5) (layer B.Cu) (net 19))
 (segment (start 20.955 28.575) (end 19.685 27.305) (width 0.5) (layer B.Cu) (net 19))
 (segment (start 54.009 22.225) (end 50.26899 25.96501) (width 0.5) (layer B.Cu) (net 19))
 (segment (start 44.7675 26.67) (end 44.7675 28.2575) (width 0.5) (layer B.Cu) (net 19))
 (segment (start 55.88 22.225) (end 54.009 22.225) (width 0.5) (layer B.Cu) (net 19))
 (segment (start 20.955 31.115) (end 20.955 28.575) (width 0.5) (layer B.Cu) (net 19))
 (segment (start 50.26899 25.96501) (end 45.47249 25.96501) (width 0.5) (layer B.Cu) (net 19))
 (segment (start 45.47249 25.96501) (end 44.7675 26.67) (width 0.5) (layer B.Cu) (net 19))
 (segment (start 44.7675 28.2575) (end 44.45 28.575) (width 0.5) (layer B.Cu) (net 19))
 (segment (start 44.45 28.575) (end 28.575 28.575) (width 0.5) (layer B.Cu) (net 19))
 (segment (start 28.575 28.575) (end 27.305 29.845) (width 0.5) (layer B.Cu) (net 19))
 (segment (start 27.305 29.845) (end 27.305 31.115) (width 0.5) (layer B.Cu) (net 19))
 (segment (start 27.305 31.115) (end 26.67 31.75) (width 0.5) (layer B.Cu) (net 19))
 (segment (start 21.59 31.75) (end 20.955 31.115) (width 0.5) (layer B.Cu) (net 19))
 (segment (start 26.67 31.75) (end 21.59 31.75) (width 0.5) (layer B.Cu) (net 19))
 (segment (start 42.545 22.225) (end 42.545 22.225) (width 0.5) (layer B.Cu) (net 20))
 (segment (start 52.705 19.685) (end 55.88 19.685) (width 0.5) (layer B.Cu) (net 20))
 (segment (start 51.435 20.955) (end 52.705 19.685) (width 0.5) (layer B.Cu) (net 20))
 (segment (start 25.4 22.225) (end 30.48 22.225) (width 0.5) (layer B.Cu) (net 20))
 (segment (start 31.75 23.495) (end 34.925 23.495) (width 0.5) (layer B.Cu) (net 20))
 (segment (start 38.1 24.13) (end 38.735 23.495) (width 0.5) (layer B.Cu) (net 20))
 (segment (start 34.925 23.495) (end 35.56 24.13) (width 0.5) (layer B.Cu) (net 20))
 (segment (start 35.56 24.13) (end 38.1 24.13) (width 0.5) (layer B.Cu) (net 20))
 (segment (start 41.91 23.495) (end 42.545 22.86) (width 0.5) (layer B.Cu) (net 20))
 (segment (start 38.735 23.495) (end 41.91 23.495) (width 0.5) (layer B.Cu) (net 20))
 (segment (start 30.48 22.225) (end 31.75 23.495) (width 0.5) (layer B.Cu) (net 20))
 (segment (start 43.18 21.59) (end 46.355 21.59) (width 0.5) (layer B.Cu) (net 20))
 (segment (start 42.545 22.86) (end 42.545 22.225) (width 0.5) (layer B.Cu) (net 20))
 (segment (start 46.355 21.59) (end 46.99 20.955) (width 0.5) (layer B.Cu) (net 20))
 (segment (start 42.545 22.225) (end 43.18 21.59) (width 0.5) (layer B.Cu) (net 20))
 (segment (start 46.99 20.955) (end 51.435 20.955) (width 0.5) (layer B.Cu) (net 20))
 (segment (start 30.48 15.875) (end 30.48 15.875) (width 0.5) (layer B.Cu) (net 21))
 (via (at 30.48 15.875) (size 1.5) (drill 0.5) (layers F.Cu B.Cu) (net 21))
 (segment (start 27.94 20.32) (end 30.48 15.875) (width 0.5) (layer F.Cu) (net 21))
 (segment (start 46.355 19.685) (end 48.26 19.685) (width 0.5) (layer B.Cu) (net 21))
 (segment (start 42.899963 20.32) (end 45.72 20.32) (width 0.5) (layer B.Cu) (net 21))
 (segment (start 42.264963 20.955) (end 42.899963 20.32) (width 0.5) (layer B.Cu) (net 21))
 (segment (start 39.37 20.955) (end 42.264963 20.955) (width 0.5) (layer B.Cu) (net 21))
 (segment (start 36.83 18.415) (end 39.37 20.955) (width 0.5) (layer B.Cu) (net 21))
 (segment (start 31.75 18.415) (end 36.83 18.415) (width 0.5) (layer B.Cu) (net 21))
 (segment (start 45.72 20.32) (end 46.355 19.685) (width 0.5) (layer B.Cu) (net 21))
 (segment (start 30.48 17.145) (end 31.75 18.415) (width 0.5) (layer B.Cu) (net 21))
 (segment (start 30.48 15.875) (end 30.48 17.145) (width 0.5) (layer B.Cu) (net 21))
 (segment (start 17.78 19.685) (end 20.32 19.685) (width 0.5) (layer B.Cu) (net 21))
 (segment (start 20.32 19.685) (end 21.59 20.955) (width 0.5) (layer B.Cu) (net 21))
 (via (at 27.94 20.32) (size 1.5) (drill 0.5) (layers F.Cu B.Cu) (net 21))
 (segment (start 27.94 20.32) (end 27.305 20.955) (width 0.5) (layer B.Cu) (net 21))
 (segment (start 21.59 20.955) (end 27.305 20.955) (width 0.5) (layer B.Cu) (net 21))
 (segment (start 23.495 29.845) (end 25.4 29.845) (width 0.5) (layer B.Cu) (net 22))
 (segment (start 22.86 29.21) (end 23.495 29.845) (width 0.5) (layer B.Cu) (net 22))
 (segment (start 22.86 26.67) (end 22.86 29.21) (width 0.5) (layer B.Cu) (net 22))
 (segment (start 23.495 26.035) (end 22.86 26.67) (width 0.5) (layer B.Cu) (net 22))
 (segment (start 47.625 22.225) (end 43.815 26.035) (width 0.5) (layer B.Cu) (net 22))
 (segment (start 48.26 22.225) (end 47.625 22.225) (width 0.5) (layer B.Cu) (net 22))
 (segment (start 34.29 26.035) (end 34.925 26.67) (width 0.5) (layer B.Cu) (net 22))
 (segment (start 34.29 26.035) (end 23.495 26.035) (width 0.5) (layer B.Cu) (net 22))
 (segment (start 34.925 26.67) (end 38.735 26.67) (width 0.5) (layer B.Cu) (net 22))
 (segment (start 38.735 26.67) (end 39.37 26.035) (width 0.5) (layer B.Cu) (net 22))
 (segment (start 43.815 26.035) (end 39.37 26.035) (width 0.5) (layer B.Cu) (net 22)))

